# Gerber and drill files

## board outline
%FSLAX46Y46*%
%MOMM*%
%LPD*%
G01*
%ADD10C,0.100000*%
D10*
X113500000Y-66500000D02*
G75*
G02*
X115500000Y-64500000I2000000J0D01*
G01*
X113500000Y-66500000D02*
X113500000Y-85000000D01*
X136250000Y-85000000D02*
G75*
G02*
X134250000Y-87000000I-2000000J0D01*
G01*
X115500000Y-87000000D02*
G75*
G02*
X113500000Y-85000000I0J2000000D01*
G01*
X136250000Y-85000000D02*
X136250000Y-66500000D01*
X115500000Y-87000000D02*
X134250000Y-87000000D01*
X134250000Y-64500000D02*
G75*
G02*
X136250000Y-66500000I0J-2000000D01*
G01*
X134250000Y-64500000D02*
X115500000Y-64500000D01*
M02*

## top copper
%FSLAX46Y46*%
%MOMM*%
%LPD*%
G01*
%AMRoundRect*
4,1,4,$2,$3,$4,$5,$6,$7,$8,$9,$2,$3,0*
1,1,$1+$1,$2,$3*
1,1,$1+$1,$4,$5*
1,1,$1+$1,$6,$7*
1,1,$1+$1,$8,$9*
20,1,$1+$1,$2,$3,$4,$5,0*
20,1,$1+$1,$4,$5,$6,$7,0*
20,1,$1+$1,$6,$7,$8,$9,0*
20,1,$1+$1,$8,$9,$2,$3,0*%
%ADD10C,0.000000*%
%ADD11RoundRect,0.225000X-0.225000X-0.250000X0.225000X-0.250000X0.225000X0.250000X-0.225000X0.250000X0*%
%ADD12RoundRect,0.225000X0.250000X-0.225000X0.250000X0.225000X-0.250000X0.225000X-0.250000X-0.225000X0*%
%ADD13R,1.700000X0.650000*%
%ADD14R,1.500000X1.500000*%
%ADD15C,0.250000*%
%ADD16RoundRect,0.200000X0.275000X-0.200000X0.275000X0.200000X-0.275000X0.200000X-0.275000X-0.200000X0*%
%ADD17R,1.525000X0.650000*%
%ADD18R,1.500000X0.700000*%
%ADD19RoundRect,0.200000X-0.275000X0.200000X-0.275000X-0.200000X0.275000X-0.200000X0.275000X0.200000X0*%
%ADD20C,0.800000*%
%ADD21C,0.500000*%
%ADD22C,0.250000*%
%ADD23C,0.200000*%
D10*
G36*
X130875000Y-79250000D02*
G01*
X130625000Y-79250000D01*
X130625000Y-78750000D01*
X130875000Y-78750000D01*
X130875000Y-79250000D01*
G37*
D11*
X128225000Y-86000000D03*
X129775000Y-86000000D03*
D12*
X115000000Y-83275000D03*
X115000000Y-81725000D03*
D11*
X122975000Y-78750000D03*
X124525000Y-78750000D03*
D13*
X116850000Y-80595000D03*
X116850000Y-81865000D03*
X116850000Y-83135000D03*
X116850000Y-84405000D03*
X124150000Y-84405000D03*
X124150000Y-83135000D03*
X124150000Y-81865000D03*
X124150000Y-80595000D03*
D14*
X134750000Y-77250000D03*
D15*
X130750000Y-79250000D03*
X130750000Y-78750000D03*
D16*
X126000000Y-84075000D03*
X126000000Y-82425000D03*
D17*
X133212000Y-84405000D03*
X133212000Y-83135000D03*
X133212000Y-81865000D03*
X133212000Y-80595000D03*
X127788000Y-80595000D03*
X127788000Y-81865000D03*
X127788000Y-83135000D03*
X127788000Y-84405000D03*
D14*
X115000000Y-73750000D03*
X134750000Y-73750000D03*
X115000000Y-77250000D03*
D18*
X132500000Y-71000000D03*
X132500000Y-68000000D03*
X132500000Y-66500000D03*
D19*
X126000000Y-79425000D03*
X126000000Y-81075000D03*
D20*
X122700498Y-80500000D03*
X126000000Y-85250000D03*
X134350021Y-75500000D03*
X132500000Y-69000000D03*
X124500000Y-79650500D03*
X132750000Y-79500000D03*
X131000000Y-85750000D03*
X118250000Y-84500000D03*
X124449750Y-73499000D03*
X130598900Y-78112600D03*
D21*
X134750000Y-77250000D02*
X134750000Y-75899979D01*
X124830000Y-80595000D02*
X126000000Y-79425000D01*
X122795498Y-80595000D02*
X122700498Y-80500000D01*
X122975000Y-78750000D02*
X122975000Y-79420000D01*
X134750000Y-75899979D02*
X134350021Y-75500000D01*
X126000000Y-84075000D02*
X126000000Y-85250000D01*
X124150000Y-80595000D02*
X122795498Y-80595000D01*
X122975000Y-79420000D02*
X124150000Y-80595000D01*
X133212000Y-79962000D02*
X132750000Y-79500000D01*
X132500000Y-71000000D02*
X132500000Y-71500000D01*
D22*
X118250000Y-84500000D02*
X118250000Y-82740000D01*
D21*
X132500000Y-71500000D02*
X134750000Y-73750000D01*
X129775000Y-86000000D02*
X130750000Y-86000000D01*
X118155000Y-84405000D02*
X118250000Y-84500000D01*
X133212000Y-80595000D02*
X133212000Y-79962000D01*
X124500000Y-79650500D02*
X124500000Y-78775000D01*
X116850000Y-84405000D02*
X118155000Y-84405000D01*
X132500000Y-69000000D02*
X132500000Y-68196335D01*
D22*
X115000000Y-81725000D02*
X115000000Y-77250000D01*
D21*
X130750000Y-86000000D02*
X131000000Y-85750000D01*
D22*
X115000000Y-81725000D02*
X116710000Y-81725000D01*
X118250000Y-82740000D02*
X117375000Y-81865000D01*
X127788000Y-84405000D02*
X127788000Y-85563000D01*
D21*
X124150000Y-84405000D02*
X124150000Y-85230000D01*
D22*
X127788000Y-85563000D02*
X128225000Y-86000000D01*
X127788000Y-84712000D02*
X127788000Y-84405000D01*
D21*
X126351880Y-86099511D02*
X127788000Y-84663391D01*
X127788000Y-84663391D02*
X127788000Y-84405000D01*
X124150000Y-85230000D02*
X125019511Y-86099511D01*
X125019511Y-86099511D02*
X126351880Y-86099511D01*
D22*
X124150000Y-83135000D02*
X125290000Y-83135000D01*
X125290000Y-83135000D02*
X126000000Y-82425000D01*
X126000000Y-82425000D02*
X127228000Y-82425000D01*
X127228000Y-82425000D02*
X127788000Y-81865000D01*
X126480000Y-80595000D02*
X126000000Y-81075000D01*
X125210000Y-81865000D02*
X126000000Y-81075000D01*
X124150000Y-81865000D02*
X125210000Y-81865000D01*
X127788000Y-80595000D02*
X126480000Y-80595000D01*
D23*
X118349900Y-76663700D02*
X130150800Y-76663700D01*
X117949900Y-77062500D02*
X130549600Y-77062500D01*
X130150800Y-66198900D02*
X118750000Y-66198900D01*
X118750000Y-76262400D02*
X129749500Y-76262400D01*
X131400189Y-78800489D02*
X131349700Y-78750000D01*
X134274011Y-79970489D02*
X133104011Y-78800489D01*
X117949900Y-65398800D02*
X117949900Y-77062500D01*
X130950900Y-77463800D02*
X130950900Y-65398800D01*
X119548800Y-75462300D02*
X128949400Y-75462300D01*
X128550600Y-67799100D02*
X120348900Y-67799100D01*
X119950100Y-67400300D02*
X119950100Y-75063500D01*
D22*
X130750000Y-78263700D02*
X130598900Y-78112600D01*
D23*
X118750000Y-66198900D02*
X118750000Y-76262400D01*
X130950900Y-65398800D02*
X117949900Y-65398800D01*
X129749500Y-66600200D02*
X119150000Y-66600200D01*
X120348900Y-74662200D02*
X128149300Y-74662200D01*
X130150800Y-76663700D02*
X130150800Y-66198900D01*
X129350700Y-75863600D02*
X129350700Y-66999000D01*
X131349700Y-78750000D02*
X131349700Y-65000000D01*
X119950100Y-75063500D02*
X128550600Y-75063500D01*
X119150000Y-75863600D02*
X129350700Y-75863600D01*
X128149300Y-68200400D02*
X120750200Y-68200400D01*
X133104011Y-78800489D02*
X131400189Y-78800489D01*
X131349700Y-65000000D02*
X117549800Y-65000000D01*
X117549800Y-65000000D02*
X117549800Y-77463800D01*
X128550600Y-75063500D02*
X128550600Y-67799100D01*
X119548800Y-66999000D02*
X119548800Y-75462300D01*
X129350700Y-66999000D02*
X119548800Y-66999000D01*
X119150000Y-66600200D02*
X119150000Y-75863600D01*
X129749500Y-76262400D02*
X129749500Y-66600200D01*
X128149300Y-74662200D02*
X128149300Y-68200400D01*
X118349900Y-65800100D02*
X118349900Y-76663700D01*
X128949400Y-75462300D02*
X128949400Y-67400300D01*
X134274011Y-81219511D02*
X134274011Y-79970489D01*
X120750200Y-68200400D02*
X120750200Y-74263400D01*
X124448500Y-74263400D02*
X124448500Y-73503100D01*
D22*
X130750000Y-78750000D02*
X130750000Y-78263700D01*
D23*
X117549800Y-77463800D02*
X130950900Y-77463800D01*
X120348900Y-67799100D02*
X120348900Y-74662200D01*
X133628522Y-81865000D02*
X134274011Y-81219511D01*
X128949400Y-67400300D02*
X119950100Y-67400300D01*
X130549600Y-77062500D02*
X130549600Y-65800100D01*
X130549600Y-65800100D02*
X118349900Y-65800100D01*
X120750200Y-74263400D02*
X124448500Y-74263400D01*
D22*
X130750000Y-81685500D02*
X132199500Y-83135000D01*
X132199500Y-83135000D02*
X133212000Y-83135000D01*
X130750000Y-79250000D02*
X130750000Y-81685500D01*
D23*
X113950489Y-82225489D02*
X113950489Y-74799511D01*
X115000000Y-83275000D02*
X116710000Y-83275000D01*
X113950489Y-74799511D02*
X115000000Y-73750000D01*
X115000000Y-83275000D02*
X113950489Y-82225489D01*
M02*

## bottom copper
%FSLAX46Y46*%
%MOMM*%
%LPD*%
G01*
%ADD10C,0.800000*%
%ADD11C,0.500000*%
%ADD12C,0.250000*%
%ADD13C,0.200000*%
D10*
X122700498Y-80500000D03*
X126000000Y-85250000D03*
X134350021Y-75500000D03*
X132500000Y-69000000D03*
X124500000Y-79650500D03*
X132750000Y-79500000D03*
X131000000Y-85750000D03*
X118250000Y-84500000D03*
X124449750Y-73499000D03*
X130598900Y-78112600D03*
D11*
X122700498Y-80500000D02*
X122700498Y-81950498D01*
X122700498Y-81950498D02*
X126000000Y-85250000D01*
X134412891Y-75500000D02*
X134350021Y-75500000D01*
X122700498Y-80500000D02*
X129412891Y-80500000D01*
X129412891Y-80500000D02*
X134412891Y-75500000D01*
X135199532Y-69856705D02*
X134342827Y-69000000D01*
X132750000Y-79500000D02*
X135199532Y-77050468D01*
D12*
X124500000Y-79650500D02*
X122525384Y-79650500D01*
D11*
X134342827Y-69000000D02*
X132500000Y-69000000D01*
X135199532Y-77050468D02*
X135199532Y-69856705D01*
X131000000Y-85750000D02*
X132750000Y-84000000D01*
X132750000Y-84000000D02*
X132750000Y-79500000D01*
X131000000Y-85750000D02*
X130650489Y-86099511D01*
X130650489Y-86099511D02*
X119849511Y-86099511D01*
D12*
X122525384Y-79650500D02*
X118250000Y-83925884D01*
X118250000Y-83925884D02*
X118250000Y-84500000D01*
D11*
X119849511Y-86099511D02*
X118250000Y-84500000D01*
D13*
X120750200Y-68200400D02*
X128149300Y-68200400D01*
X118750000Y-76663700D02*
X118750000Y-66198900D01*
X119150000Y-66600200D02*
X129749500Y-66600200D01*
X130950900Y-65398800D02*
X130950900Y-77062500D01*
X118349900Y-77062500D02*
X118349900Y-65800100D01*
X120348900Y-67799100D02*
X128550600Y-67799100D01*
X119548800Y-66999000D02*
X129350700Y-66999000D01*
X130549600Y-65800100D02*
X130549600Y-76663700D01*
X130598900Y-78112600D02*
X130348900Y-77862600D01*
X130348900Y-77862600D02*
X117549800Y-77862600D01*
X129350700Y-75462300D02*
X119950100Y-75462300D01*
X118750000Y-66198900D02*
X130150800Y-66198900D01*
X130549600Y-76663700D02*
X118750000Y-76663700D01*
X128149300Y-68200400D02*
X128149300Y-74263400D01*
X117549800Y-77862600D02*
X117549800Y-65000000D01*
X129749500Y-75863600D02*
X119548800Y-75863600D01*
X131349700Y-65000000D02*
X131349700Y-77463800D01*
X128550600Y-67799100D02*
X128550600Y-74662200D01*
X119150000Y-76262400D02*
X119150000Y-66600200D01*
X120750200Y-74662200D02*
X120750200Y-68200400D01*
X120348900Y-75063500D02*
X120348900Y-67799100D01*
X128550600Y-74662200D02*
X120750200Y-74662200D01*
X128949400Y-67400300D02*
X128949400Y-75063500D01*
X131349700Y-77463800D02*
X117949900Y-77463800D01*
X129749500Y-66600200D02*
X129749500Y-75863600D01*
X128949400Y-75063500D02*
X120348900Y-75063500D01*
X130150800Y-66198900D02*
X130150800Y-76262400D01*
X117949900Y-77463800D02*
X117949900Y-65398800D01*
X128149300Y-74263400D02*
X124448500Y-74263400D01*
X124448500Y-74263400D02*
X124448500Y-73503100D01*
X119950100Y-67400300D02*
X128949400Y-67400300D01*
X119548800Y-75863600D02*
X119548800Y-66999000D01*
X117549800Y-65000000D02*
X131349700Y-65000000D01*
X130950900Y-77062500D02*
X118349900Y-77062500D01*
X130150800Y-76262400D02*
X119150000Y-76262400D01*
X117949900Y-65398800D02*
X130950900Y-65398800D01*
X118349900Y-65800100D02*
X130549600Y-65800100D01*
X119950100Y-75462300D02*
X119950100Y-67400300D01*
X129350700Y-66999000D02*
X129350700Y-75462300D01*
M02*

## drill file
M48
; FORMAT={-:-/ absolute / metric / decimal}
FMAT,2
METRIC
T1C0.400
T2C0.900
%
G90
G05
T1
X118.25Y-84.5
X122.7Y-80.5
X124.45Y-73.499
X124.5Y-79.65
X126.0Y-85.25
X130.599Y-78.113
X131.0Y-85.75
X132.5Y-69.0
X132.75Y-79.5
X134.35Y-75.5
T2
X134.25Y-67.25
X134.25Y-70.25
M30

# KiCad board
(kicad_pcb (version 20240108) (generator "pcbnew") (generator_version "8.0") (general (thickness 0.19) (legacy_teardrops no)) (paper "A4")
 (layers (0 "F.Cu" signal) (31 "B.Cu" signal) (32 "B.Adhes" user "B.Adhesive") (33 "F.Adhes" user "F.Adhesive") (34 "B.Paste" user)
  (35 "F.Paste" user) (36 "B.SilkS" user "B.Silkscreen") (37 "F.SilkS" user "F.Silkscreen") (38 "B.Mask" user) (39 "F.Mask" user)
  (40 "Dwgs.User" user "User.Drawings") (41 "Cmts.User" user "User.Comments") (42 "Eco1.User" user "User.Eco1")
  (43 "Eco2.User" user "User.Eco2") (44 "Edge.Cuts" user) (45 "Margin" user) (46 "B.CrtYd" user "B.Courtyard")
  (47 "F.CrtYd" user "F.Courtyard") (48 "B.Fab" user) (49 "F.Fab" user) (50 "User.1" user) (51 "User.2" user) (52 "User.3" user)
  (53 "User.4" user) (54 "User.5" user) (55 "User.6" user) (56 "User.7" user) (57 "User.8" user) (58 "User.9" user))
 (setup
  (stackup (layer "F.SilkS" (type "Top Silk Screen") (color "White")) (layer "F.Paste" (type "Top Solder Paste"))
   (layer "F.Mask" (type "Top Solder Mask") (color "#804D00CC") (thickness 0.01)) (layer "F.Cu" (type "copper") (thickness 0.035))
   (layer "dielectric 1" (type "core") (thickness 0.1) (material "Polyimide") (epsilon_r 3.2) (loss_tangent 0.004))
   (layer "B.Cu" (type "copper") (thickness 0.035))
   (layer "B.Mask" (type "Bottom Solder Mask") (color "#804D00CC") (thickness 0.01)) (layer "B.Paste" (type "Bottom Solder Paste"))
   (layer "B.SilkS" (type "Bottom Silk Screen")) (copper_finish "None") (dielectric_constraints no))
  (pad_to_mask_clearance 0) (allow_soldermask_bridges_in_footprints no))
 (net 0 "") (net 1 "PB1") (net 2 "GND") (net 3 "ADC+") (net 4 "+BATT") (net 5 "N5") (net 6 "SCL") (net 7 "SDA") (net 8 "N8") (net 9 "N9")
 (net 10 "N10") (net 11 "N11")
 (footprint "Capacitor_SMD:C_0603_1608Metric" (layer "F.Cu") (at 129 86)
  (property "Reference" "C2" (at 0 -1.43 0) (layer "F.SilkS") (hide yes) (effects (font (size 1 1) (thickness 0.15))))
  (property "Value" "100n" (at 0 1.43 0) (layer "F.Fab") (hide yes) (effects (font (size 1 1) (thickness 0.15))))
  (pad "1" smd roundrect (at -0.775 0) (size 0.9 0.95) (layers "F.Cu" "F.Paste" "F.Mask") (roundrect_rratio 0.25) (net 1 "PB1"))
  (pad "2" smd roundrect (at 0.775 0) (size 0.9 0.95) (layers "F.Cu" "F.Paste" "F.Mask") (roundrect_rratio 0.25) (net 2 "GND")))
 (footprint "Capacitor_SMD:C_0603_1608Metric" (layer "F.Cu") (at 115 82.5 90)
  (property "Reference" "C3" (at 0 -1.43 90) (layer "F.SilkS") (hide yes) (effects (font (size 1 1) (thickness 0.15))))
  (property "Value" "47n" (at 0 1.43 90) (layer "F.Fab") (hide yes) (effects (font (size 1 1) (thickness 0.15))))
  (pad "1" smd roundrect (at -0.775 0 90) (size 0.9 0.95) (layers "F.Cu" "F.Paste" "F.Mask") (roundrect_rratio 0.25) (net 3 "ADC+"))
  (pad "2" smd roundrect (at 0.775 0 90) (size 0.9 0.95) (layers "F.Cu" "F.Paste" "F.Mask") (roundrect_rratio 0.25) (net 2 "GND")))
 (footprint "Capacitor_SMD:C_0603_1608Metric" (layer "F.Cu") (at 123.75 78.75)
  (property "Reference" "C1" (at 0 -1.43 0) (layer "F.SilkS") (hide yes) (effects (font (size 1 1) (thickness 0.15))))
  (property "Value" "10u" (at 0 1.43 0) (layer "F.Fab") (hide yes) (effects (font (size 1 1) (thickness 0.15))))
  (pad "1" smd roundrect (at -0.775 0) (size 0.9 0.95) (layers "F.Cu" "F.Paste" "F.Mask") (roundrect_rratio 0.25) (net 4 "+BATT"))
  (pad "2" smd roundrect (at 0.775 0) (size 0.9 0.95) (layers "F.Cu" "F.Paste" "F.Mask") (roundrect_rratio 0.25) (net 2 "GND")))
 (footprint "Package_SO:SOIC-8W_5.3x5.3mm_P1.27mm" (layer "F.Cu") (at 120.5 82.5)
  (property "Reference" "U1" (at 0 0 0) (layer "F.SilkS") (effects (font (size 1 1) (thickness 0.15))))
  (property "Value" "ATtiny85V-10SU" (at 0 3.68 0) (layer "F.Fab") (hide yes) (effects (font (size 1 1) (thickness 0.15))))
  (pad "1" smd rect (at -3.65 -1.905) (size 1.7 0.65) (layers "F.Cu" "F.Paste" "F.Mask") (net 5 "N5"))
  (pad "2" smd rect (at -3.65 -0.635) (size 1.7 0.65) (layers "F.Cu" "F.Paste" "F.Mask") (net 2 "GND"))
  (pad "3" smd rect (at -3.65 0.635) (size 1.7 0.65) (layers "F.Cu" "F.Paste" "F.Mask") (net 3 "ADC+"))
  (pad "4" smd rect (at -3.65 1.905) (size 1.7 0.65) (layers "F.Cu" "F.Paste" "F.Mask") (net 2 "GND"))
  (pad "5" smd rect (at 3.65 1.905) (size 1.7 0.65) (layers "F.Cu" "F.Paste" "F.Mask") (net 1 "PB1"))
  (pad "6" smd rect (at 3.65 0.635) (size 1.7 0.65) (layers "F.Cu" "F.Paste" "F.Mask") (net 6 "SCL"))
  (pad "7" smd rect (at 3.65 -0.635) (size 1.7 0.65) (layers "F.Cu" "F.Paste" "F.Mask") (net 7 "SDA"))
  (pad "8" smd rect (at 3.65 -1.905) (size 1.7 0.65) (layers "F.Cu" "F.Paste" "F.Mask") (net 4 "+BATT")))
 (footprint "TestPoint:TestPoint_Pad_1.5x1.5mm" (layer "F.Cu") (at 134.75 77.25 90)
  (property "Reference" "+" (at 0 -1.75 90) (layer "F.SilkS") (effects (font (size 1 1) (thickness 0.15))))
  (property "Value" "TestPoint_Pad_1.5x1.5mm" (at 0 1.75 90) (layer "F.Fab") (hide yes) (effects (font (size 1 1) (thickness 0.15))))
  (pad "1" smd rect (at 0 0 90) (size 1.5 1.5) (layers "F.Cu" "F.Mask") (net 4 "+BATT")))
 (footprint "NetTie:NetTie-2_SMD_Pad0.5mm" (layer "F.Cu") (at 130.75 79.25 90)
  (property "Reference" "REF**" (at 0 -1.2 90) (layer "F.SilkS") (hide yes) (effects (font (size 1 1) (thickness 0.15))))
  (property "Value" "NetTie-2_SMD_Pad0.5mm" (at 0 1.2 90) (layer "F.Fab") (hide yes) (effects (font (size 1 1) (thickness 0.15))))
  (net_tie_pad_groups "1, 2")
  (fp_poly (pts (xy 0 -0.125) (xy 0.5 -0.125) (xy 0.5 0.125) (xy 0 0.125)) (stroke (width 0) (type solid)) (fill solid) (layer "F.Cu"))
  (pad "1" smd circle (at 0 0 90) (size 0.25 0.25) (layers "F.Cu") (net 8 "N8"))
  (pad "2" smd circle (at 0.5 0 90) (size 0.25 0.25) (layers "F.Cu") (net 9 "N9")))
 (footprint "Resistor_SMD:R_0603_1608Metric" (layer "F.Cu") (at 126 83.25 90)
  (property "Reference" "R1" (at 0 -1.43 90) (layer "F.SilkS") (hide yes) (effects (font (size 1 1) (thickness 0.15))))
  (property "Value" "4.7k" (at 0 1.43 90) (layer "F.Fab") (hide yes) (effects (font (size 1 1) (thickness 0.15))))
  (pad "1" smd roundrect (at -0.825 0 90) (size 0.8 0.95) (layers "F.Cu" "F.Paste" "F.Mask") (roundrect_rratio 0.25) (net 4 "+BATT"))
  (pad "2" smd roundrect (at 0.825 0 90) (size 0.8 0.95) (layers "F.Cu" "F.Paste" "F.Mask") (roundrect_rratio 0.25) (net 6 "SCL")))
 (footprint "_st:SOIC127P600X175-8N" (layer "F.Cu") (at 130.5 82.5 180)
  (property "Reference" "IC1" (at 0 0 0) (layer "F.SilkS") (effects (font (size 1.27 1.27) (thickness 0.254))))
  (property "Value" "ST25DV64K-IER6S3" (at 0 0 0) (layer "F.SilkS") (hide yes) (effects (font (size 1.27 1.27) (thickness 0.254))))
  (pad "1" smd rect (at -2.712 -1.905 270) (size 0.65 1.525) (layers "F.Cu" "F.Paste" "F.Mask") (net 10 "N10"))
  (pad "2" smd rect (at -2.712 -0.635 270) (size 0.65 1.525) (layers "F.Cu" "F.Paste" "F.Mask") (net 8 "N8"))
  (pad "3" smd rect (at -2.712 0.635 270) (size 0.65 1.525) (layers "F.Cu" "F.Paste" "F.Mask") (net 9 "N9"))
  (pad "4" smd rect (at -2.712 1.905 270) (size 0.65 1.525) (layers "F.Cu" "F.Paste" "F.Mask") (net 2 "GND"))
  (pad "5" smd rect (at 2.712 1.905 270) (size 0.65 1.525) (layers "F.Cu" "F.Paste" "F.Mask") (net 7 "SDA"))
  (pad "6" smd rect (at 2.712 0.635 270) (size 0.65 1.525) (layers "F.Cu" "F.Paste" "F.Mask") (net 6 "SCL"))
  (pad "7" smd rect (at 2.712 -0.635 270) (size 0.65 1.525) (layers "F.Cu" "F.Paste" "F.Mask") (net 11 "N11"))
  (pad "8" smd rect (at 2.712 -1.905 270) (size 0.65 1.525) (layers "F.Cu" "F.Paste" "F.Mask") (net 1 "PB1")))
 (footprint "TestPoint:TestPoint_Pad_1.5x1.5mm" (layer "F.Cu") (at 115 73.75 -90)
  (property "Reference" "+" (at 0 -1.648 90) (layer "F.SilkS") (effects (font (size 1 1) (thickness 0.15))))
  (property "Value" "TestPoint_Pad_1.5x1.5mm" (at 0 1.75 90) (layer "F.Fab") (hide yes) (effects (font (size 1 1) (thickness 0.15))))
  (pad "1" smd rect (at 0 0 270) (size 1.5 1.5) (layers "F.Cu" "F.Mask") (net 3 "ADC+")))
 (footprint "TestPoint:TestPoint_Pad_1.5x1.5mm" (layer "F.Cu") (at 134.75 73.75 90)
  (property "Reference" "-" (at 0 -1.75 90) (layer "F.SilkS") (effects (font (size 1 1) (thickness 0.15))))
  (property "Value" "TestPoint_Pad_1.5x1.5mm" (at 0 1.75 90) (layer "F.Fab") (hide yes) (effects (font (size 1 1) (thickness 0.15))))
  (pad "1" smd rect (at 0 0 90) (size 1.5 1.5) (layers "F.Cu" "F.Mask") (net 2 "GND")))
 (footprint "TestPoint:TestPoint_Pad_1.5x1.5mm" (layer "F.Cu") (at 115 77.25 -90)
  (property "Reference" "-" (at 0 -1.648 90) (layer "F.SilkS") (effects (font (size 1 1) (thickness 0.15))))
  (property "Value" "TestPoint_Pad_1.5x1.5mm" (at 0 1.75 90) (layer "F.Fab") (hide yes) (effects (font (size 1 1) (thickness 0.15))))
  (pad "1" smd rect (at 0 0 270) (size 1.5 1.5) (layers "F.Cu" "F.Mask") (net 2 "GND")))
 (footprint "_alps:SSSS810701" (layer "F.Cu") (at 132.5 68 90)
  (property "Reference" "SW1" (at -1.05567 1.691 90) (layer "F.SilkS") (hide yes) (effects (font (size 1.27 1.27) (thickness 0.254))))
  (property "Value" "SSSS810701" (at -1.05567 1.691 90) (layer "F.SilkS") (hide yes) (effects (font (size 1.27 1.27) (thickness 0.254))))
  (pad "" np_thru_hole circle (at -2.25 1.75 90) (size 0.9 0.9) (drill 0.9) (layers "*.Cu" "*.Mask"))
  (pad "" np_thru_hole circle (at 0.75 1.75 90) (size 0.9 0.9) (drill 0.9) (layers "*.Cu" "*.Mask"))
  (pad "1" smd rect (at -3 0 90) (size 0.7 1.5) (layers "F.Cu" "F.Paste" "F.Mask") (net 2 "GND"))
  (pad "2" smd rect (at 0 0 90) (size 0.7 1.5) (layers "F.Cu" "F.Paste" "F.Mask") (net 2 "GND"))
  (pad "3" smd rect (at 1.5 0 90) (size 0.7 1.5) (layers "F.Cu" "F.Paste" "F.Mask")))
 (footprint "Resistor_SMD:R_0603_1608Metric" (layer "F.Cu") (at 126 80.25 -90)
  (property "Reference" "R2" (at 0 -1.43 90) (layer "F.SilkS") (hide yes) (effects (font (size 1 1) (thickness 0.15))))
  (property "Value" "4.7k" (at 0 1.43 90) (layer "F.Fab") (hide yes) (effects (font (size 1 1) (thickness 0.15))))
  (pad "1" smd roundrect (at -0.825 0 270) (size 0.8 0.95) (layers "F.Cu" "F.Paste" "F.Mask") (roundrect_rratio 0.25) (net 4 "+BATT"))
  (pad "2" smd roundrect (at 0.825 0 270) (size 0.8 0.95) (layers "F.Cu" "F.Paste" "F.Mask") (roundrect_rratio 0.25) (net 7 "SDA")))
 (gr_arc (start 113.5 66.5) (mid 114.085786 65.085786) (end 115.5 64.5) (stroke (width 0.1) (type solid)) (layer "Edge.Cuts"))
 (gr_line (start 113.5 66.5) (end 113.5 85) (stroke (width 0.1) (type solid)) (layer "Edge.Cuts"))
 (gr_arc (start 136.25 85) (mid 135.664214 86.414214) (end 134.25 87) (stroke (width 0.1) (type solid)) (layer "Edge.Cuts"))
 (gr_arc (start 115.5 87) (mid 114.085786 86.414214) (end 113.5 85) (stroke (width 0.1) (type solid)) (layer "Edge.Cuts"))
 (gr_line (start 136.25 85) (end 136.25 66.5) (stroke (width 0.1) (type solid)) (layer "Edge.Cuts"))
 (gr_line (start 115.5 87) (end 134.25 87) (stroke (width 0.1) (type solid)) (layer "Edge.Cuts"))
 (gr_arc (start 134.25 64.5) (mid 135.664214 65.085786) (end 136.25 66.5) (stroke (width 0.1) (type solid)) (layer "Edge.Cuts"))
 (gr_line (start 134.25 64.5) (end 115.5 64.5) (stroke (width 0.1) (type solid)) (layer "Edge.Cuts"))
 (segment (start 134.75 77.25) (end 134.75 75.899979) (width 0.5) (layer "F.Cu") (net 4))
 (segment (start 124.83 80.595) (end 126 79.425) (width 0.5) (layer "F.Cu") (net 4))
 (segment (start 122.795498 80.595) (end 122.700498 80.5) (width 0.5) (layer "F.Cu") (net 4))
 (segment (start 122.975 78.75) (end 122.975 79.42) (width 0.5) (layer "F.Cu") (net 4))
 (segment (start 134.75 75.899979) (end 134.350021 75.5) (width 0.5) (layer "F.Cu") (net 4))
 (segment (start 126 84.075) (end 126 85.25) (width 0.5) (layer "F.Cu") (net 4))
 (segment (start 124.15 80.595) (end 122.795498 80.595) (width 0.5) (layer "F.Cu") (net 4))
 (segment (start 122.975 79.42) (end 124.15 80.595) (width 0.5) (layer "F.Cu") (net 4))
 (via (at 122.700498 80.5) (size 0.8) (drill 0.4) (layers "F.Cu" "B.Cu") (free yes) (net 4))
 (via (at 126 85.25) (size 0.8) (drill 0.4) (layers "F.Cu" "B.Cu") (free yes) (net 4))
 (via (at 134.350021 75.5) (size 0.8) (drill 0.4) (layers "F.Cu" "B.Cu") (free yes) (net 4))
 (segment (start 122.700498 80.5) (end 122.700498 81.950498) (width 0.5) (layer "B.Cu") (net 4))
 (segment (start 122.700498 81.950498) (end 126 85.25) (width 0.5) (layer "B.Cu") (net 4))
 (segment (start 134.412891 75.5) (end 134.350021 75.5) (width 0.5) (layer "B.Cu") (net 4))
 (segment (start 122.700498 80.5) (end 129.412891 80.5) (width 0.5) (layer "B.Cu") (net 4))
 (segment (start 129.412891 80.5) (end 134.412891 75.5) (width 0.5) (layer "B.Cu") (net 4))
 (segment (start 133.212 79.962) (end 132.75 79.5) (width 0.5) (layer "F.Cu") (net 2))
 (segment (start 132.5 71) (end 132.5 71.5) (width 0.5) (layer "F.Cu") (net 2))
 (segment (start 118.25 84.5) (end 118.25 82.74) (width 0.25) (layer "F.Cu") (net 2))
 (segment (start 132.5 71.5) (end 134.75 73.75) (width 0.5) (layer "F.Cu") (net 2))
 (segment (start 129.775 86) (end 130.75 86) (width 0.5) (layer "F.Cu") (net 2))
 (segment (start 118.155 84.405) (end 118.25 84.5) (width 0.5) (layer "F.Cu") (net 2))
 (segment (start 133.212 80.595) (end 133.212 79.962) (width 0.5) (layer "F.Cu") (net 2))
 (segment (start 124.5 79.6505) (end 124.5 78.775) (width 0.5) (layer "F.Cu") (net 2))
 (segment (start 116.85 84.405) (end 118.155 84.405) (width 0.5) (layer "F.Cu") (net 2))
 (segment (start 132.5 69) (end 132.5 68.196335) (width 0.5) (layer "F.Cu") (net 2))
 (segment (start 115 81.725) (end 115 77.25) (width 0.25) (layer "F.Cu") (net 2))
 (segment (start 130.75 86) (end 131 85.75) (width 0.5) (layer "F.Cu") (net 2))
 (segment (start 115 81.725) (end 116.71 81.725) (width 0.25) (layer "F.Cu") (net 2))
 (segment (start 118.25 82.74) (end 117.375 81.865) (width 0.25) (layer "F.Cu") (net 2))
 (via (at 132.5 69) (size 0.8) (drill 0.4) (layers "F.Cu" "B.Cu") (free yes) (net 2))
 (via (at 124.5 79.6505) (size 0.8) (drill 0.4) (layers "F.Cu" "B.Cu") (free yes) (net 2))
 (via (at 132.75 79.5) (size 0.8) (drill 0.4) (layers "F.Cu" "B.Cu") (free yes) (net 2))
 (via (at 131 85.75) (size 0.8) (drill 0.4) (layers "F.Cu" "B.Cu") (free yes) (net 2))
 (via (at 118.25 84.5) (size 0.8) (drill 0.4) (layers "F.Cu" "B.Cu") (free yes) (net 2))
 (segment (start 135.199532 69.856705) (end 134.342827 69) (width 0.5) (layer "B.Cu") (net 2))
 (segment (start 132.75 79.5) (end 135.199532 77.050468) (width 0.5) (layer "B.Cu") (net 2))
 (segment (start 124.5 79.6505) (end 122.525384 79.6505) (width 0.25) (layer "B.Cu") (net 2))
 (segment (start 134.342827 69) (end 132.5 69) (width 0.5) (layer "B.Cu") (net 2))
 (segment (start 135.199532 77.050468) (end 135.199532 69.856705) (width 0.5) (layer "B.Cu") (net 2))
 (segment (start 131 85.75) (end 132.75 84) (width 0.5) (layer "B.Cu") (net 2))
 (segment (start 132.75 84) (end 132.75 79.5) (width 0.5) (layer "B.Cu") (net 2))
 (segment (start 131 85.75) (end 130.650489 86.099511) (width 0.5) (layer "B.Cu") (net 2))
 (segment (start 130.650489 86.099511) (end 119.849511 86.099511) (width 0.5) (layer "B.Cu") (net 2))
 (segment (start 122.525384 79.6505) (end 118.25 83.925884) (width 0.25) (layer "B.Cu") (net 2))
 (segment (start 118.25 83.925884) (end 118.25 84.5) (width 0.25) (layer "B.Cu") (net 2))
 (segment (start 119.849511 86.099511) (end 118.25 84.5) (width 0.5) (layer "B.Cu") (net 2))
 (segment (start 127.788 84.405) (end 127.788 85.563) (width 0.25) (layer "F.Cu") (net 1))
 (segment (start 124.15 84.405) (end 124.15 85.23) (width 0.5) (layer "F.Cu") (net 1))
 (segment (start 127.788 85.563) (end 128.225 86) (width 0.25) (layer "F.Cu") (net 1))
 (segment (start 127.788 84.712) (end 127.788 84.405) (width 0.25) (layer "F.Cu") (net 1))
 (segment (start 126.35188 86.099511) (end 127.788 84.663391) (width 0.5) (layer "F.Cu") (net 1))
 (segment (start 127.788 84.663391) (end 127.788 84.405) (width 0.5) (layer "F.Cu") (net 1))
 (segment (start 124.15 85.23) (end 125.019511 86.099511) (width 0.5) (layer "F.Cu") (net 1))
 (segment (start 125.019511 86.099511) (end 126.35188 86.099511) (width 0.5) (layer "F.Cu") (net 1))
 (segment (start 124.15 83.135) (end 125.29 83.135) (width 0.25) (layer "F.Cu") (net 6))
 (segment (start 125.29 83.135) (end 126 82.425) (width 0.25) (layer "F.Cu") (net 6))
 (segment (start 126 82.425) (end 127.228 82.425) (width 0.25) (layer "F.Cu") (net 6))
 (segment (start 127.228 82.425) (end 127.788 81.865) (width 0.25) (layer "F.Cu") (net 6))
 (segment (start 126.48 80.595) (end 126 81.075) (width 0.25) (layer "F.Cu") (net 7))
 (segment (start 125.21 81.865) (end 126 81.075) (width 0.25) (layer "F.Cu") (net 7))
 (segment (start 124.15 81.865) (end 125.21 81.865) (width 0.25) (layer "F.Cu") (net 7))
 (segment (start 127.788 80.595) (end 126.48 80.595) (width 0.25) (layer "F.Cu") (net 7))
 (segment (start 118.3499 76.6637) (end 130.1508 76.6637) (width 0.2) (layer "F.Cu") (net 9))
 (segment (start 117.9499 77.0625) (end 130.5496 77.0625) (width 0.2) (layer "F.Cu") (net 9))
 (segment (start 130.1508 66.1989) (end 118.75 66.1989) (width 0.2) (layer "F.Cu") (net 9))
 (segment (start 118.75 76.2624) (end 129.7495 76.2624) (width 0.2) (layer "F.Cu") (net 9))
 (segment (start 131.400189 78.800489) (end 131.3497 78.75) (width 0.2) (layer "F.Cu") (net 9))
 (segment (start 134.274011 79.970489) (end 133.104011 78.800489) (width 0.2) (layer "F.Cu") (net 9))
 (segment (start 117.9499 65.3988) (end 117.9499 77.0625) (width 0.2) (layer "F.Cu") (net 9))
 (segment (start 130.9509 77.4638) (end 130.9509 65.3988) (width 0.2) (layer "F.Cu") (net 9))
 (segment (start 119.5488 75.4623) (end 128.9494 75.4623) (width 0.2) (layer "F.Cu") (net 9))
 (segment (start 128.5506 67.7991) (end 120.3489 67.7991) (width 0.2) (layer "F.Cu") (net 9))
 (segment (start 119.9501 67.4003) (end 119.9501 75.0635) (width 0.2) (layer "F.Cu") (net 9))
 (segment (start 130.75 78.2637) (end 130.5989 78.1126) (width 0.25) (layer "F.Cu") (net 9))
 (segment (start 118.75 66.1989) (end 118.75 76.2624) (width 0.2) (layer "F.Cu") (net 9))
 (segment (start 130.9509 65.3988) (end 117.9499 65.3988) (width 0.2) (layer "F.Cu") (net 9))
 (segment (start 129.7495 66.6002) (end 119.15 66.6002) (width 0.2) (layer "F.Cu") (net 9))
 (segment (start 120.3489 74.6622) (end 128.1493 74.6622) (width 0.2) (layer "F.Cu") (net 9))
 (segment (start 130.1508 76.6637) (end 130.1508 66.1989) (width 0.2) (layer "F.Cu") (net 9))
 (segment (start 129.3507 75.8636) (end 129.3507 66.999) (width 0.2) (layer "F.Cu") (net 9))
 (segment (start 131.3497 78.75) (end 131.3497 65) (width 0.2) (layer "F.Cu") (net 9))
 (segment (start 119.9501 75.0635) (end 128.5506 75.0635) (width 0.2) (layer "F.Cu") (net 9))
 (segment (start 119.15 75.8636) (end 129.3507 75.8636) (width 0.2) (layer "F.Cu") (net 9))
 (segment (start 128.1493 68.2004) (end 120.7502 68.2004) (width 0.2) (layer "F.Cu") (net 9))
 (segment (start 133.104011 78.800489) (end 131.400189 78.800489) (width 0.2) (layer "F.Cu") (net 9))
 (segment (start 131.3497 65) (end 117.5498 65) (width 0.2) (layer "F.Cu") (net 9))
 (segment (start 117.5498 65) (end 117.5498 77.4638) (width 0.2) (layer "F.Cu") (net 9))
 (segment (start 128.5506 75.0635) (end 128.5506 67.7991) (width 0.2) (layer "F.Cu") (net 9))
 (segment (start 119.5488 66.999) (end 119.5488 75.4623) (width 0.2) (layer "F.Cu") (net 9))
 (segment (start 129.3507 66.999) (end 119.5488 66.999) (width 0.2) (layer "F.Cu") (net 9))
 (segment (start 119.15 66.6002) (end 119.15 75.8636) (width 0.2) (layer "F.Cu") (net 9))
 (segment (start 129.7495 76.2624) (end 129.7495 66.6002) (width 0.2) (layer "F.Cu") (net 9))
 (segment (start 128.1493 74.6622) (end 128.1493 68.2004) (width 0.2) (layer "F.Cu") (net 9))
 (segment (start 118.3499 65.8001) (end 118.3499 76.6637) (width 0.2) (layer "F.Cu") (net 9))
 (segment (start 128.9494 75.4623) (end 128.9494 67.4003) (width 0.2) (layer "F.Cu") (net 9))
 (segment (start 134.274011 81.219511) (end 134.274011 79.970489) (width 0.2) (layer "F.Cu") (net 9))
 (segment (start 120.7502 68.2004) (end 120.7502 74.2634) (width 0.2) (layer "F.Cu") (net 9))
 (segment (start 124.4485 74.2634) (end 124.4485 73.5031) (width 0.2) (layer "F.Cu") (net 9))
 (segment (start 130.75 78.75) (end 130.75 78.2637) (width 0.25) (layer "F.Cu") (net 9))
 (segment (start 117.5498 77.4638) (end 130.9509 77.4638) (width 0.2) (layer "F.Cu") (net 9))
 (segment (start 120.3489 67.7991) (end 120.3489 74.6622) (width 0.2) (layer "F.Cu") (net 9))
 (segment (start 133.628522 81.865) (end 134.274011 81.219511) (width 0.2) (layer "F.Cu") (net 9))
 (segment (start 128.9494 67.4003) (end 119.9501 67.4003) (width 0.2) (layer "F.Cu") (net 9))
 (segment (start 130.5496 77.0625) (end 130.5496 65.8001) (width 0.2) (layer "F.Cu") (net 9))
 (segment (start 130.5496 65.8001) (end 118.3499 65.8001) (width 0.2) (layer "F.Cu") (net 9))
 (segment (start 120.7502 74.2634) (end 124.4485 74.2634) (width 0.2) (layer "F.Cu") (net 9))
 (via (at 124.44975 73.499) (size 0.8) (drill 0.4) (layers "F.Cu" "B.Cu") (free yes) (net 9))
 (via (at 130.5989 78.1126) (size 0.8) (drill 0.4) (layers "F.Cu" "B.Cu") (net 9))
 (segment (start 120.7502 68.2004) (end 128.1493 68.2004) (width 0.2) (layer "B.Cu") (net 9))
 (segment (start 118.75 76.6637) (end 118.75 66.1989) (width 0.2) (layer "B.Cu") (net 9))
 (segment (start 119.15 66.6002) (end 129.7495 66.6002) (width 0.2) (layer "B.Cu") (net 9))
 (segment (start 130.9509 65.3988) (end 130.9509 77.0625) (width 0.2) (layer "B.Cu") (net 9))
 (segment (start 118.3499 77.0625) (end 118.3499 65.8001) (width 0.2) (layer "B.Cu") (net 9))
 (segment (start 120.3489 67.7991) (end 128.5506 67.7991) (width 0.2) (layer "B.Cu") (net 9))
 (segment (start 119.5488 66.999) (end 129.3507 66.999) (width 0.2) (layer "B.Cu") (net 9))
 (segment (start 130.5496 65.8001) (end 130.5496 76.6637) (width 0.2) (layer "B.Cu") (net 9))
 (segment (start 130.5989 78.1126) (end 130.3489 77.8626) (width 0.2) (layer "B.Cu") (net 9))
 (segment (start 130.3489 77.8626) (end 117.5498 77.8626) (width 0.2) (layer "B.Cu") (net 9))
 (segment (start 129.3507 75.4623) (end 119.9501 75.4623) (width 0.2) (layer "B.Cu") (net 9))
 (segment (start 118.75 66.1989) (end 130.1508 66.1989) (width 0.2) (layer "B.Cu") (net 9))
 (segment (start 130.5496 76.6637) (end 118.75 76.6637) (width 0.2) (layer "B.Cu") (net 9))
 (segment (start 128.1493 68.2004) (end 128.1493 74.2634) (width 0.2) (layer "B.Cu") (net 9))
 (segment (start 117.5498 77.8626) (end 117.5498 65) (width 0.2) (layer "B.Cu") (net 9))
 (segment (start 129.7495 75.8636) (end 119.5488 75.8636) (width 0.2) (layer "B.Cu") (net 9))
 (segment (start 131.3497 65) (end 131.3497 77.4638) (width 0.2) (layer "B.Cu") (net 9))
 (segment (start 128.5506 67.7991) (end 128.5506 74.6622) (width 0.2) (layer "B.Cu") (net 9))
 (segment (start 119.15 76.2624) (end 119.15 66.6002) (width 0.2) (layer "B.Cu") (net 9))
 (segment (start 120.7502 74.6622) (end 120.7502 68.2004) (width 0.2) (layer "B.Cu") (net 9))
 (segment (start 120.3489 75.0635) (end 120.3489 67.7991) (width 0.2) (layer "B.Cu") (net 9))
 (segment (start 128.5506 74.6622) (end 120.7502 74.6622) (width 0.2) (layer "B.Cu") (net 9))
 (segment (start 128.9494 67.4003) (end 128.9494 75.0635) (width 0.2) (layer "B.Cu") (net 9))
 (segment (start 131.3497 77.4638) (end 117.9499 77.4638) (width 0.2) (layer "B.Cu") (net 9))
 (segment (start 129.7495 66.6002) (end 129.7495 75.8636) (width 0.2) (layer "B.Cu") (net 9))
 (segment (start 128.9494 75.0635) (end 120.3489 75.0635) (width 0.2) (layer "B.Cu") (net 9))
 (segment (start 130.1508 66.1989) (end 130.1508 76.2624) (width 0.2) (layer "B.Cu") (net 9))
 (segment (start 117.9499 77.4638) (end 117.9499 65.3988) (width 0.2) (layer "B.Cu") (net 9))
 (segment (start 128.1493 74.2634) (end 124.4485 74.2634) (width 0.2) (layer "B.Cu") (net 9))
 (segment (start 124.4485 74.2634) (end 124.4485 73.5031) (width 0.2) (layer "B.Cu") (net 9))
 (segment (start 119.9501 67.4003) (end 128.9494 67.4003) (width 0.2) (layer "B.Cu") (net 9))
 (segment (start 119.5488 75.8636) (end 119.5488 66.999) (width 0.2) (layer "B.Cu") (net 9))
 (segment (start 117.5498 65) (end 131.3497 65) (width 0.2) (layer "B.Cu") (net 9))
 (segment (start 130.9509 77.0625) (end 118.3499 77.0625) (width 0.2) (layer "B.Cu") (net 9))
 (segment (start 130.1508 76.2624) (end 119.15 76.2624) (width 0.2) (layer "B.Cu") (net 9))
 (segment (start 117.9499 65.3988) (end 130.9509 65.3988) (width 0.2) (layer "B.Cu") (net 9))
 (segment (start 118.3499 65.8001) (end 130.5496 65.8001) (width 0.2) (layer "B.Cu") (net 9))
 (segment (start 119.9501 75.4623) (end 119.9501 67.4003) (width 0.2) (layer "B.Cu") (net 9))
 (segment (start 129.3507 66.999) (end 129.3507 75.4623) (width 0.2) (layer "B.Cu") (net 9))
 (segment (start 130.75 81.6855) (end 132.1995 83.135) (width 0.25) (layer "F.Cu") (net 8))
 (segment (start 132.1995 83.135) (end 133.212 83.135) (width 0.25) (layer "F.Cu") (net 8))
 (segment (start 130.75 79.25) (end 130.75 81.6855) (width 0.25) (layer "F.Cu") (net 8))
 (segment (start 113.950489 82.225489) (end 113.950489 74.799511) (width 0.2) (layer "F.Cu") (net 3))
 (segment (start 115 83.275) (end 116.71 83.275) (width 0.2) (layer "F.Cu") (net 3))
 (segment (start 113.950489 74.799511) (end 115 73.75) (width 0.2) (layer "F.Cu") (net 3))
 (segment (start 115 83.275) (end 113.950489 82.225489) (width 0.2) (layer "F.Cu") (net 3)))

